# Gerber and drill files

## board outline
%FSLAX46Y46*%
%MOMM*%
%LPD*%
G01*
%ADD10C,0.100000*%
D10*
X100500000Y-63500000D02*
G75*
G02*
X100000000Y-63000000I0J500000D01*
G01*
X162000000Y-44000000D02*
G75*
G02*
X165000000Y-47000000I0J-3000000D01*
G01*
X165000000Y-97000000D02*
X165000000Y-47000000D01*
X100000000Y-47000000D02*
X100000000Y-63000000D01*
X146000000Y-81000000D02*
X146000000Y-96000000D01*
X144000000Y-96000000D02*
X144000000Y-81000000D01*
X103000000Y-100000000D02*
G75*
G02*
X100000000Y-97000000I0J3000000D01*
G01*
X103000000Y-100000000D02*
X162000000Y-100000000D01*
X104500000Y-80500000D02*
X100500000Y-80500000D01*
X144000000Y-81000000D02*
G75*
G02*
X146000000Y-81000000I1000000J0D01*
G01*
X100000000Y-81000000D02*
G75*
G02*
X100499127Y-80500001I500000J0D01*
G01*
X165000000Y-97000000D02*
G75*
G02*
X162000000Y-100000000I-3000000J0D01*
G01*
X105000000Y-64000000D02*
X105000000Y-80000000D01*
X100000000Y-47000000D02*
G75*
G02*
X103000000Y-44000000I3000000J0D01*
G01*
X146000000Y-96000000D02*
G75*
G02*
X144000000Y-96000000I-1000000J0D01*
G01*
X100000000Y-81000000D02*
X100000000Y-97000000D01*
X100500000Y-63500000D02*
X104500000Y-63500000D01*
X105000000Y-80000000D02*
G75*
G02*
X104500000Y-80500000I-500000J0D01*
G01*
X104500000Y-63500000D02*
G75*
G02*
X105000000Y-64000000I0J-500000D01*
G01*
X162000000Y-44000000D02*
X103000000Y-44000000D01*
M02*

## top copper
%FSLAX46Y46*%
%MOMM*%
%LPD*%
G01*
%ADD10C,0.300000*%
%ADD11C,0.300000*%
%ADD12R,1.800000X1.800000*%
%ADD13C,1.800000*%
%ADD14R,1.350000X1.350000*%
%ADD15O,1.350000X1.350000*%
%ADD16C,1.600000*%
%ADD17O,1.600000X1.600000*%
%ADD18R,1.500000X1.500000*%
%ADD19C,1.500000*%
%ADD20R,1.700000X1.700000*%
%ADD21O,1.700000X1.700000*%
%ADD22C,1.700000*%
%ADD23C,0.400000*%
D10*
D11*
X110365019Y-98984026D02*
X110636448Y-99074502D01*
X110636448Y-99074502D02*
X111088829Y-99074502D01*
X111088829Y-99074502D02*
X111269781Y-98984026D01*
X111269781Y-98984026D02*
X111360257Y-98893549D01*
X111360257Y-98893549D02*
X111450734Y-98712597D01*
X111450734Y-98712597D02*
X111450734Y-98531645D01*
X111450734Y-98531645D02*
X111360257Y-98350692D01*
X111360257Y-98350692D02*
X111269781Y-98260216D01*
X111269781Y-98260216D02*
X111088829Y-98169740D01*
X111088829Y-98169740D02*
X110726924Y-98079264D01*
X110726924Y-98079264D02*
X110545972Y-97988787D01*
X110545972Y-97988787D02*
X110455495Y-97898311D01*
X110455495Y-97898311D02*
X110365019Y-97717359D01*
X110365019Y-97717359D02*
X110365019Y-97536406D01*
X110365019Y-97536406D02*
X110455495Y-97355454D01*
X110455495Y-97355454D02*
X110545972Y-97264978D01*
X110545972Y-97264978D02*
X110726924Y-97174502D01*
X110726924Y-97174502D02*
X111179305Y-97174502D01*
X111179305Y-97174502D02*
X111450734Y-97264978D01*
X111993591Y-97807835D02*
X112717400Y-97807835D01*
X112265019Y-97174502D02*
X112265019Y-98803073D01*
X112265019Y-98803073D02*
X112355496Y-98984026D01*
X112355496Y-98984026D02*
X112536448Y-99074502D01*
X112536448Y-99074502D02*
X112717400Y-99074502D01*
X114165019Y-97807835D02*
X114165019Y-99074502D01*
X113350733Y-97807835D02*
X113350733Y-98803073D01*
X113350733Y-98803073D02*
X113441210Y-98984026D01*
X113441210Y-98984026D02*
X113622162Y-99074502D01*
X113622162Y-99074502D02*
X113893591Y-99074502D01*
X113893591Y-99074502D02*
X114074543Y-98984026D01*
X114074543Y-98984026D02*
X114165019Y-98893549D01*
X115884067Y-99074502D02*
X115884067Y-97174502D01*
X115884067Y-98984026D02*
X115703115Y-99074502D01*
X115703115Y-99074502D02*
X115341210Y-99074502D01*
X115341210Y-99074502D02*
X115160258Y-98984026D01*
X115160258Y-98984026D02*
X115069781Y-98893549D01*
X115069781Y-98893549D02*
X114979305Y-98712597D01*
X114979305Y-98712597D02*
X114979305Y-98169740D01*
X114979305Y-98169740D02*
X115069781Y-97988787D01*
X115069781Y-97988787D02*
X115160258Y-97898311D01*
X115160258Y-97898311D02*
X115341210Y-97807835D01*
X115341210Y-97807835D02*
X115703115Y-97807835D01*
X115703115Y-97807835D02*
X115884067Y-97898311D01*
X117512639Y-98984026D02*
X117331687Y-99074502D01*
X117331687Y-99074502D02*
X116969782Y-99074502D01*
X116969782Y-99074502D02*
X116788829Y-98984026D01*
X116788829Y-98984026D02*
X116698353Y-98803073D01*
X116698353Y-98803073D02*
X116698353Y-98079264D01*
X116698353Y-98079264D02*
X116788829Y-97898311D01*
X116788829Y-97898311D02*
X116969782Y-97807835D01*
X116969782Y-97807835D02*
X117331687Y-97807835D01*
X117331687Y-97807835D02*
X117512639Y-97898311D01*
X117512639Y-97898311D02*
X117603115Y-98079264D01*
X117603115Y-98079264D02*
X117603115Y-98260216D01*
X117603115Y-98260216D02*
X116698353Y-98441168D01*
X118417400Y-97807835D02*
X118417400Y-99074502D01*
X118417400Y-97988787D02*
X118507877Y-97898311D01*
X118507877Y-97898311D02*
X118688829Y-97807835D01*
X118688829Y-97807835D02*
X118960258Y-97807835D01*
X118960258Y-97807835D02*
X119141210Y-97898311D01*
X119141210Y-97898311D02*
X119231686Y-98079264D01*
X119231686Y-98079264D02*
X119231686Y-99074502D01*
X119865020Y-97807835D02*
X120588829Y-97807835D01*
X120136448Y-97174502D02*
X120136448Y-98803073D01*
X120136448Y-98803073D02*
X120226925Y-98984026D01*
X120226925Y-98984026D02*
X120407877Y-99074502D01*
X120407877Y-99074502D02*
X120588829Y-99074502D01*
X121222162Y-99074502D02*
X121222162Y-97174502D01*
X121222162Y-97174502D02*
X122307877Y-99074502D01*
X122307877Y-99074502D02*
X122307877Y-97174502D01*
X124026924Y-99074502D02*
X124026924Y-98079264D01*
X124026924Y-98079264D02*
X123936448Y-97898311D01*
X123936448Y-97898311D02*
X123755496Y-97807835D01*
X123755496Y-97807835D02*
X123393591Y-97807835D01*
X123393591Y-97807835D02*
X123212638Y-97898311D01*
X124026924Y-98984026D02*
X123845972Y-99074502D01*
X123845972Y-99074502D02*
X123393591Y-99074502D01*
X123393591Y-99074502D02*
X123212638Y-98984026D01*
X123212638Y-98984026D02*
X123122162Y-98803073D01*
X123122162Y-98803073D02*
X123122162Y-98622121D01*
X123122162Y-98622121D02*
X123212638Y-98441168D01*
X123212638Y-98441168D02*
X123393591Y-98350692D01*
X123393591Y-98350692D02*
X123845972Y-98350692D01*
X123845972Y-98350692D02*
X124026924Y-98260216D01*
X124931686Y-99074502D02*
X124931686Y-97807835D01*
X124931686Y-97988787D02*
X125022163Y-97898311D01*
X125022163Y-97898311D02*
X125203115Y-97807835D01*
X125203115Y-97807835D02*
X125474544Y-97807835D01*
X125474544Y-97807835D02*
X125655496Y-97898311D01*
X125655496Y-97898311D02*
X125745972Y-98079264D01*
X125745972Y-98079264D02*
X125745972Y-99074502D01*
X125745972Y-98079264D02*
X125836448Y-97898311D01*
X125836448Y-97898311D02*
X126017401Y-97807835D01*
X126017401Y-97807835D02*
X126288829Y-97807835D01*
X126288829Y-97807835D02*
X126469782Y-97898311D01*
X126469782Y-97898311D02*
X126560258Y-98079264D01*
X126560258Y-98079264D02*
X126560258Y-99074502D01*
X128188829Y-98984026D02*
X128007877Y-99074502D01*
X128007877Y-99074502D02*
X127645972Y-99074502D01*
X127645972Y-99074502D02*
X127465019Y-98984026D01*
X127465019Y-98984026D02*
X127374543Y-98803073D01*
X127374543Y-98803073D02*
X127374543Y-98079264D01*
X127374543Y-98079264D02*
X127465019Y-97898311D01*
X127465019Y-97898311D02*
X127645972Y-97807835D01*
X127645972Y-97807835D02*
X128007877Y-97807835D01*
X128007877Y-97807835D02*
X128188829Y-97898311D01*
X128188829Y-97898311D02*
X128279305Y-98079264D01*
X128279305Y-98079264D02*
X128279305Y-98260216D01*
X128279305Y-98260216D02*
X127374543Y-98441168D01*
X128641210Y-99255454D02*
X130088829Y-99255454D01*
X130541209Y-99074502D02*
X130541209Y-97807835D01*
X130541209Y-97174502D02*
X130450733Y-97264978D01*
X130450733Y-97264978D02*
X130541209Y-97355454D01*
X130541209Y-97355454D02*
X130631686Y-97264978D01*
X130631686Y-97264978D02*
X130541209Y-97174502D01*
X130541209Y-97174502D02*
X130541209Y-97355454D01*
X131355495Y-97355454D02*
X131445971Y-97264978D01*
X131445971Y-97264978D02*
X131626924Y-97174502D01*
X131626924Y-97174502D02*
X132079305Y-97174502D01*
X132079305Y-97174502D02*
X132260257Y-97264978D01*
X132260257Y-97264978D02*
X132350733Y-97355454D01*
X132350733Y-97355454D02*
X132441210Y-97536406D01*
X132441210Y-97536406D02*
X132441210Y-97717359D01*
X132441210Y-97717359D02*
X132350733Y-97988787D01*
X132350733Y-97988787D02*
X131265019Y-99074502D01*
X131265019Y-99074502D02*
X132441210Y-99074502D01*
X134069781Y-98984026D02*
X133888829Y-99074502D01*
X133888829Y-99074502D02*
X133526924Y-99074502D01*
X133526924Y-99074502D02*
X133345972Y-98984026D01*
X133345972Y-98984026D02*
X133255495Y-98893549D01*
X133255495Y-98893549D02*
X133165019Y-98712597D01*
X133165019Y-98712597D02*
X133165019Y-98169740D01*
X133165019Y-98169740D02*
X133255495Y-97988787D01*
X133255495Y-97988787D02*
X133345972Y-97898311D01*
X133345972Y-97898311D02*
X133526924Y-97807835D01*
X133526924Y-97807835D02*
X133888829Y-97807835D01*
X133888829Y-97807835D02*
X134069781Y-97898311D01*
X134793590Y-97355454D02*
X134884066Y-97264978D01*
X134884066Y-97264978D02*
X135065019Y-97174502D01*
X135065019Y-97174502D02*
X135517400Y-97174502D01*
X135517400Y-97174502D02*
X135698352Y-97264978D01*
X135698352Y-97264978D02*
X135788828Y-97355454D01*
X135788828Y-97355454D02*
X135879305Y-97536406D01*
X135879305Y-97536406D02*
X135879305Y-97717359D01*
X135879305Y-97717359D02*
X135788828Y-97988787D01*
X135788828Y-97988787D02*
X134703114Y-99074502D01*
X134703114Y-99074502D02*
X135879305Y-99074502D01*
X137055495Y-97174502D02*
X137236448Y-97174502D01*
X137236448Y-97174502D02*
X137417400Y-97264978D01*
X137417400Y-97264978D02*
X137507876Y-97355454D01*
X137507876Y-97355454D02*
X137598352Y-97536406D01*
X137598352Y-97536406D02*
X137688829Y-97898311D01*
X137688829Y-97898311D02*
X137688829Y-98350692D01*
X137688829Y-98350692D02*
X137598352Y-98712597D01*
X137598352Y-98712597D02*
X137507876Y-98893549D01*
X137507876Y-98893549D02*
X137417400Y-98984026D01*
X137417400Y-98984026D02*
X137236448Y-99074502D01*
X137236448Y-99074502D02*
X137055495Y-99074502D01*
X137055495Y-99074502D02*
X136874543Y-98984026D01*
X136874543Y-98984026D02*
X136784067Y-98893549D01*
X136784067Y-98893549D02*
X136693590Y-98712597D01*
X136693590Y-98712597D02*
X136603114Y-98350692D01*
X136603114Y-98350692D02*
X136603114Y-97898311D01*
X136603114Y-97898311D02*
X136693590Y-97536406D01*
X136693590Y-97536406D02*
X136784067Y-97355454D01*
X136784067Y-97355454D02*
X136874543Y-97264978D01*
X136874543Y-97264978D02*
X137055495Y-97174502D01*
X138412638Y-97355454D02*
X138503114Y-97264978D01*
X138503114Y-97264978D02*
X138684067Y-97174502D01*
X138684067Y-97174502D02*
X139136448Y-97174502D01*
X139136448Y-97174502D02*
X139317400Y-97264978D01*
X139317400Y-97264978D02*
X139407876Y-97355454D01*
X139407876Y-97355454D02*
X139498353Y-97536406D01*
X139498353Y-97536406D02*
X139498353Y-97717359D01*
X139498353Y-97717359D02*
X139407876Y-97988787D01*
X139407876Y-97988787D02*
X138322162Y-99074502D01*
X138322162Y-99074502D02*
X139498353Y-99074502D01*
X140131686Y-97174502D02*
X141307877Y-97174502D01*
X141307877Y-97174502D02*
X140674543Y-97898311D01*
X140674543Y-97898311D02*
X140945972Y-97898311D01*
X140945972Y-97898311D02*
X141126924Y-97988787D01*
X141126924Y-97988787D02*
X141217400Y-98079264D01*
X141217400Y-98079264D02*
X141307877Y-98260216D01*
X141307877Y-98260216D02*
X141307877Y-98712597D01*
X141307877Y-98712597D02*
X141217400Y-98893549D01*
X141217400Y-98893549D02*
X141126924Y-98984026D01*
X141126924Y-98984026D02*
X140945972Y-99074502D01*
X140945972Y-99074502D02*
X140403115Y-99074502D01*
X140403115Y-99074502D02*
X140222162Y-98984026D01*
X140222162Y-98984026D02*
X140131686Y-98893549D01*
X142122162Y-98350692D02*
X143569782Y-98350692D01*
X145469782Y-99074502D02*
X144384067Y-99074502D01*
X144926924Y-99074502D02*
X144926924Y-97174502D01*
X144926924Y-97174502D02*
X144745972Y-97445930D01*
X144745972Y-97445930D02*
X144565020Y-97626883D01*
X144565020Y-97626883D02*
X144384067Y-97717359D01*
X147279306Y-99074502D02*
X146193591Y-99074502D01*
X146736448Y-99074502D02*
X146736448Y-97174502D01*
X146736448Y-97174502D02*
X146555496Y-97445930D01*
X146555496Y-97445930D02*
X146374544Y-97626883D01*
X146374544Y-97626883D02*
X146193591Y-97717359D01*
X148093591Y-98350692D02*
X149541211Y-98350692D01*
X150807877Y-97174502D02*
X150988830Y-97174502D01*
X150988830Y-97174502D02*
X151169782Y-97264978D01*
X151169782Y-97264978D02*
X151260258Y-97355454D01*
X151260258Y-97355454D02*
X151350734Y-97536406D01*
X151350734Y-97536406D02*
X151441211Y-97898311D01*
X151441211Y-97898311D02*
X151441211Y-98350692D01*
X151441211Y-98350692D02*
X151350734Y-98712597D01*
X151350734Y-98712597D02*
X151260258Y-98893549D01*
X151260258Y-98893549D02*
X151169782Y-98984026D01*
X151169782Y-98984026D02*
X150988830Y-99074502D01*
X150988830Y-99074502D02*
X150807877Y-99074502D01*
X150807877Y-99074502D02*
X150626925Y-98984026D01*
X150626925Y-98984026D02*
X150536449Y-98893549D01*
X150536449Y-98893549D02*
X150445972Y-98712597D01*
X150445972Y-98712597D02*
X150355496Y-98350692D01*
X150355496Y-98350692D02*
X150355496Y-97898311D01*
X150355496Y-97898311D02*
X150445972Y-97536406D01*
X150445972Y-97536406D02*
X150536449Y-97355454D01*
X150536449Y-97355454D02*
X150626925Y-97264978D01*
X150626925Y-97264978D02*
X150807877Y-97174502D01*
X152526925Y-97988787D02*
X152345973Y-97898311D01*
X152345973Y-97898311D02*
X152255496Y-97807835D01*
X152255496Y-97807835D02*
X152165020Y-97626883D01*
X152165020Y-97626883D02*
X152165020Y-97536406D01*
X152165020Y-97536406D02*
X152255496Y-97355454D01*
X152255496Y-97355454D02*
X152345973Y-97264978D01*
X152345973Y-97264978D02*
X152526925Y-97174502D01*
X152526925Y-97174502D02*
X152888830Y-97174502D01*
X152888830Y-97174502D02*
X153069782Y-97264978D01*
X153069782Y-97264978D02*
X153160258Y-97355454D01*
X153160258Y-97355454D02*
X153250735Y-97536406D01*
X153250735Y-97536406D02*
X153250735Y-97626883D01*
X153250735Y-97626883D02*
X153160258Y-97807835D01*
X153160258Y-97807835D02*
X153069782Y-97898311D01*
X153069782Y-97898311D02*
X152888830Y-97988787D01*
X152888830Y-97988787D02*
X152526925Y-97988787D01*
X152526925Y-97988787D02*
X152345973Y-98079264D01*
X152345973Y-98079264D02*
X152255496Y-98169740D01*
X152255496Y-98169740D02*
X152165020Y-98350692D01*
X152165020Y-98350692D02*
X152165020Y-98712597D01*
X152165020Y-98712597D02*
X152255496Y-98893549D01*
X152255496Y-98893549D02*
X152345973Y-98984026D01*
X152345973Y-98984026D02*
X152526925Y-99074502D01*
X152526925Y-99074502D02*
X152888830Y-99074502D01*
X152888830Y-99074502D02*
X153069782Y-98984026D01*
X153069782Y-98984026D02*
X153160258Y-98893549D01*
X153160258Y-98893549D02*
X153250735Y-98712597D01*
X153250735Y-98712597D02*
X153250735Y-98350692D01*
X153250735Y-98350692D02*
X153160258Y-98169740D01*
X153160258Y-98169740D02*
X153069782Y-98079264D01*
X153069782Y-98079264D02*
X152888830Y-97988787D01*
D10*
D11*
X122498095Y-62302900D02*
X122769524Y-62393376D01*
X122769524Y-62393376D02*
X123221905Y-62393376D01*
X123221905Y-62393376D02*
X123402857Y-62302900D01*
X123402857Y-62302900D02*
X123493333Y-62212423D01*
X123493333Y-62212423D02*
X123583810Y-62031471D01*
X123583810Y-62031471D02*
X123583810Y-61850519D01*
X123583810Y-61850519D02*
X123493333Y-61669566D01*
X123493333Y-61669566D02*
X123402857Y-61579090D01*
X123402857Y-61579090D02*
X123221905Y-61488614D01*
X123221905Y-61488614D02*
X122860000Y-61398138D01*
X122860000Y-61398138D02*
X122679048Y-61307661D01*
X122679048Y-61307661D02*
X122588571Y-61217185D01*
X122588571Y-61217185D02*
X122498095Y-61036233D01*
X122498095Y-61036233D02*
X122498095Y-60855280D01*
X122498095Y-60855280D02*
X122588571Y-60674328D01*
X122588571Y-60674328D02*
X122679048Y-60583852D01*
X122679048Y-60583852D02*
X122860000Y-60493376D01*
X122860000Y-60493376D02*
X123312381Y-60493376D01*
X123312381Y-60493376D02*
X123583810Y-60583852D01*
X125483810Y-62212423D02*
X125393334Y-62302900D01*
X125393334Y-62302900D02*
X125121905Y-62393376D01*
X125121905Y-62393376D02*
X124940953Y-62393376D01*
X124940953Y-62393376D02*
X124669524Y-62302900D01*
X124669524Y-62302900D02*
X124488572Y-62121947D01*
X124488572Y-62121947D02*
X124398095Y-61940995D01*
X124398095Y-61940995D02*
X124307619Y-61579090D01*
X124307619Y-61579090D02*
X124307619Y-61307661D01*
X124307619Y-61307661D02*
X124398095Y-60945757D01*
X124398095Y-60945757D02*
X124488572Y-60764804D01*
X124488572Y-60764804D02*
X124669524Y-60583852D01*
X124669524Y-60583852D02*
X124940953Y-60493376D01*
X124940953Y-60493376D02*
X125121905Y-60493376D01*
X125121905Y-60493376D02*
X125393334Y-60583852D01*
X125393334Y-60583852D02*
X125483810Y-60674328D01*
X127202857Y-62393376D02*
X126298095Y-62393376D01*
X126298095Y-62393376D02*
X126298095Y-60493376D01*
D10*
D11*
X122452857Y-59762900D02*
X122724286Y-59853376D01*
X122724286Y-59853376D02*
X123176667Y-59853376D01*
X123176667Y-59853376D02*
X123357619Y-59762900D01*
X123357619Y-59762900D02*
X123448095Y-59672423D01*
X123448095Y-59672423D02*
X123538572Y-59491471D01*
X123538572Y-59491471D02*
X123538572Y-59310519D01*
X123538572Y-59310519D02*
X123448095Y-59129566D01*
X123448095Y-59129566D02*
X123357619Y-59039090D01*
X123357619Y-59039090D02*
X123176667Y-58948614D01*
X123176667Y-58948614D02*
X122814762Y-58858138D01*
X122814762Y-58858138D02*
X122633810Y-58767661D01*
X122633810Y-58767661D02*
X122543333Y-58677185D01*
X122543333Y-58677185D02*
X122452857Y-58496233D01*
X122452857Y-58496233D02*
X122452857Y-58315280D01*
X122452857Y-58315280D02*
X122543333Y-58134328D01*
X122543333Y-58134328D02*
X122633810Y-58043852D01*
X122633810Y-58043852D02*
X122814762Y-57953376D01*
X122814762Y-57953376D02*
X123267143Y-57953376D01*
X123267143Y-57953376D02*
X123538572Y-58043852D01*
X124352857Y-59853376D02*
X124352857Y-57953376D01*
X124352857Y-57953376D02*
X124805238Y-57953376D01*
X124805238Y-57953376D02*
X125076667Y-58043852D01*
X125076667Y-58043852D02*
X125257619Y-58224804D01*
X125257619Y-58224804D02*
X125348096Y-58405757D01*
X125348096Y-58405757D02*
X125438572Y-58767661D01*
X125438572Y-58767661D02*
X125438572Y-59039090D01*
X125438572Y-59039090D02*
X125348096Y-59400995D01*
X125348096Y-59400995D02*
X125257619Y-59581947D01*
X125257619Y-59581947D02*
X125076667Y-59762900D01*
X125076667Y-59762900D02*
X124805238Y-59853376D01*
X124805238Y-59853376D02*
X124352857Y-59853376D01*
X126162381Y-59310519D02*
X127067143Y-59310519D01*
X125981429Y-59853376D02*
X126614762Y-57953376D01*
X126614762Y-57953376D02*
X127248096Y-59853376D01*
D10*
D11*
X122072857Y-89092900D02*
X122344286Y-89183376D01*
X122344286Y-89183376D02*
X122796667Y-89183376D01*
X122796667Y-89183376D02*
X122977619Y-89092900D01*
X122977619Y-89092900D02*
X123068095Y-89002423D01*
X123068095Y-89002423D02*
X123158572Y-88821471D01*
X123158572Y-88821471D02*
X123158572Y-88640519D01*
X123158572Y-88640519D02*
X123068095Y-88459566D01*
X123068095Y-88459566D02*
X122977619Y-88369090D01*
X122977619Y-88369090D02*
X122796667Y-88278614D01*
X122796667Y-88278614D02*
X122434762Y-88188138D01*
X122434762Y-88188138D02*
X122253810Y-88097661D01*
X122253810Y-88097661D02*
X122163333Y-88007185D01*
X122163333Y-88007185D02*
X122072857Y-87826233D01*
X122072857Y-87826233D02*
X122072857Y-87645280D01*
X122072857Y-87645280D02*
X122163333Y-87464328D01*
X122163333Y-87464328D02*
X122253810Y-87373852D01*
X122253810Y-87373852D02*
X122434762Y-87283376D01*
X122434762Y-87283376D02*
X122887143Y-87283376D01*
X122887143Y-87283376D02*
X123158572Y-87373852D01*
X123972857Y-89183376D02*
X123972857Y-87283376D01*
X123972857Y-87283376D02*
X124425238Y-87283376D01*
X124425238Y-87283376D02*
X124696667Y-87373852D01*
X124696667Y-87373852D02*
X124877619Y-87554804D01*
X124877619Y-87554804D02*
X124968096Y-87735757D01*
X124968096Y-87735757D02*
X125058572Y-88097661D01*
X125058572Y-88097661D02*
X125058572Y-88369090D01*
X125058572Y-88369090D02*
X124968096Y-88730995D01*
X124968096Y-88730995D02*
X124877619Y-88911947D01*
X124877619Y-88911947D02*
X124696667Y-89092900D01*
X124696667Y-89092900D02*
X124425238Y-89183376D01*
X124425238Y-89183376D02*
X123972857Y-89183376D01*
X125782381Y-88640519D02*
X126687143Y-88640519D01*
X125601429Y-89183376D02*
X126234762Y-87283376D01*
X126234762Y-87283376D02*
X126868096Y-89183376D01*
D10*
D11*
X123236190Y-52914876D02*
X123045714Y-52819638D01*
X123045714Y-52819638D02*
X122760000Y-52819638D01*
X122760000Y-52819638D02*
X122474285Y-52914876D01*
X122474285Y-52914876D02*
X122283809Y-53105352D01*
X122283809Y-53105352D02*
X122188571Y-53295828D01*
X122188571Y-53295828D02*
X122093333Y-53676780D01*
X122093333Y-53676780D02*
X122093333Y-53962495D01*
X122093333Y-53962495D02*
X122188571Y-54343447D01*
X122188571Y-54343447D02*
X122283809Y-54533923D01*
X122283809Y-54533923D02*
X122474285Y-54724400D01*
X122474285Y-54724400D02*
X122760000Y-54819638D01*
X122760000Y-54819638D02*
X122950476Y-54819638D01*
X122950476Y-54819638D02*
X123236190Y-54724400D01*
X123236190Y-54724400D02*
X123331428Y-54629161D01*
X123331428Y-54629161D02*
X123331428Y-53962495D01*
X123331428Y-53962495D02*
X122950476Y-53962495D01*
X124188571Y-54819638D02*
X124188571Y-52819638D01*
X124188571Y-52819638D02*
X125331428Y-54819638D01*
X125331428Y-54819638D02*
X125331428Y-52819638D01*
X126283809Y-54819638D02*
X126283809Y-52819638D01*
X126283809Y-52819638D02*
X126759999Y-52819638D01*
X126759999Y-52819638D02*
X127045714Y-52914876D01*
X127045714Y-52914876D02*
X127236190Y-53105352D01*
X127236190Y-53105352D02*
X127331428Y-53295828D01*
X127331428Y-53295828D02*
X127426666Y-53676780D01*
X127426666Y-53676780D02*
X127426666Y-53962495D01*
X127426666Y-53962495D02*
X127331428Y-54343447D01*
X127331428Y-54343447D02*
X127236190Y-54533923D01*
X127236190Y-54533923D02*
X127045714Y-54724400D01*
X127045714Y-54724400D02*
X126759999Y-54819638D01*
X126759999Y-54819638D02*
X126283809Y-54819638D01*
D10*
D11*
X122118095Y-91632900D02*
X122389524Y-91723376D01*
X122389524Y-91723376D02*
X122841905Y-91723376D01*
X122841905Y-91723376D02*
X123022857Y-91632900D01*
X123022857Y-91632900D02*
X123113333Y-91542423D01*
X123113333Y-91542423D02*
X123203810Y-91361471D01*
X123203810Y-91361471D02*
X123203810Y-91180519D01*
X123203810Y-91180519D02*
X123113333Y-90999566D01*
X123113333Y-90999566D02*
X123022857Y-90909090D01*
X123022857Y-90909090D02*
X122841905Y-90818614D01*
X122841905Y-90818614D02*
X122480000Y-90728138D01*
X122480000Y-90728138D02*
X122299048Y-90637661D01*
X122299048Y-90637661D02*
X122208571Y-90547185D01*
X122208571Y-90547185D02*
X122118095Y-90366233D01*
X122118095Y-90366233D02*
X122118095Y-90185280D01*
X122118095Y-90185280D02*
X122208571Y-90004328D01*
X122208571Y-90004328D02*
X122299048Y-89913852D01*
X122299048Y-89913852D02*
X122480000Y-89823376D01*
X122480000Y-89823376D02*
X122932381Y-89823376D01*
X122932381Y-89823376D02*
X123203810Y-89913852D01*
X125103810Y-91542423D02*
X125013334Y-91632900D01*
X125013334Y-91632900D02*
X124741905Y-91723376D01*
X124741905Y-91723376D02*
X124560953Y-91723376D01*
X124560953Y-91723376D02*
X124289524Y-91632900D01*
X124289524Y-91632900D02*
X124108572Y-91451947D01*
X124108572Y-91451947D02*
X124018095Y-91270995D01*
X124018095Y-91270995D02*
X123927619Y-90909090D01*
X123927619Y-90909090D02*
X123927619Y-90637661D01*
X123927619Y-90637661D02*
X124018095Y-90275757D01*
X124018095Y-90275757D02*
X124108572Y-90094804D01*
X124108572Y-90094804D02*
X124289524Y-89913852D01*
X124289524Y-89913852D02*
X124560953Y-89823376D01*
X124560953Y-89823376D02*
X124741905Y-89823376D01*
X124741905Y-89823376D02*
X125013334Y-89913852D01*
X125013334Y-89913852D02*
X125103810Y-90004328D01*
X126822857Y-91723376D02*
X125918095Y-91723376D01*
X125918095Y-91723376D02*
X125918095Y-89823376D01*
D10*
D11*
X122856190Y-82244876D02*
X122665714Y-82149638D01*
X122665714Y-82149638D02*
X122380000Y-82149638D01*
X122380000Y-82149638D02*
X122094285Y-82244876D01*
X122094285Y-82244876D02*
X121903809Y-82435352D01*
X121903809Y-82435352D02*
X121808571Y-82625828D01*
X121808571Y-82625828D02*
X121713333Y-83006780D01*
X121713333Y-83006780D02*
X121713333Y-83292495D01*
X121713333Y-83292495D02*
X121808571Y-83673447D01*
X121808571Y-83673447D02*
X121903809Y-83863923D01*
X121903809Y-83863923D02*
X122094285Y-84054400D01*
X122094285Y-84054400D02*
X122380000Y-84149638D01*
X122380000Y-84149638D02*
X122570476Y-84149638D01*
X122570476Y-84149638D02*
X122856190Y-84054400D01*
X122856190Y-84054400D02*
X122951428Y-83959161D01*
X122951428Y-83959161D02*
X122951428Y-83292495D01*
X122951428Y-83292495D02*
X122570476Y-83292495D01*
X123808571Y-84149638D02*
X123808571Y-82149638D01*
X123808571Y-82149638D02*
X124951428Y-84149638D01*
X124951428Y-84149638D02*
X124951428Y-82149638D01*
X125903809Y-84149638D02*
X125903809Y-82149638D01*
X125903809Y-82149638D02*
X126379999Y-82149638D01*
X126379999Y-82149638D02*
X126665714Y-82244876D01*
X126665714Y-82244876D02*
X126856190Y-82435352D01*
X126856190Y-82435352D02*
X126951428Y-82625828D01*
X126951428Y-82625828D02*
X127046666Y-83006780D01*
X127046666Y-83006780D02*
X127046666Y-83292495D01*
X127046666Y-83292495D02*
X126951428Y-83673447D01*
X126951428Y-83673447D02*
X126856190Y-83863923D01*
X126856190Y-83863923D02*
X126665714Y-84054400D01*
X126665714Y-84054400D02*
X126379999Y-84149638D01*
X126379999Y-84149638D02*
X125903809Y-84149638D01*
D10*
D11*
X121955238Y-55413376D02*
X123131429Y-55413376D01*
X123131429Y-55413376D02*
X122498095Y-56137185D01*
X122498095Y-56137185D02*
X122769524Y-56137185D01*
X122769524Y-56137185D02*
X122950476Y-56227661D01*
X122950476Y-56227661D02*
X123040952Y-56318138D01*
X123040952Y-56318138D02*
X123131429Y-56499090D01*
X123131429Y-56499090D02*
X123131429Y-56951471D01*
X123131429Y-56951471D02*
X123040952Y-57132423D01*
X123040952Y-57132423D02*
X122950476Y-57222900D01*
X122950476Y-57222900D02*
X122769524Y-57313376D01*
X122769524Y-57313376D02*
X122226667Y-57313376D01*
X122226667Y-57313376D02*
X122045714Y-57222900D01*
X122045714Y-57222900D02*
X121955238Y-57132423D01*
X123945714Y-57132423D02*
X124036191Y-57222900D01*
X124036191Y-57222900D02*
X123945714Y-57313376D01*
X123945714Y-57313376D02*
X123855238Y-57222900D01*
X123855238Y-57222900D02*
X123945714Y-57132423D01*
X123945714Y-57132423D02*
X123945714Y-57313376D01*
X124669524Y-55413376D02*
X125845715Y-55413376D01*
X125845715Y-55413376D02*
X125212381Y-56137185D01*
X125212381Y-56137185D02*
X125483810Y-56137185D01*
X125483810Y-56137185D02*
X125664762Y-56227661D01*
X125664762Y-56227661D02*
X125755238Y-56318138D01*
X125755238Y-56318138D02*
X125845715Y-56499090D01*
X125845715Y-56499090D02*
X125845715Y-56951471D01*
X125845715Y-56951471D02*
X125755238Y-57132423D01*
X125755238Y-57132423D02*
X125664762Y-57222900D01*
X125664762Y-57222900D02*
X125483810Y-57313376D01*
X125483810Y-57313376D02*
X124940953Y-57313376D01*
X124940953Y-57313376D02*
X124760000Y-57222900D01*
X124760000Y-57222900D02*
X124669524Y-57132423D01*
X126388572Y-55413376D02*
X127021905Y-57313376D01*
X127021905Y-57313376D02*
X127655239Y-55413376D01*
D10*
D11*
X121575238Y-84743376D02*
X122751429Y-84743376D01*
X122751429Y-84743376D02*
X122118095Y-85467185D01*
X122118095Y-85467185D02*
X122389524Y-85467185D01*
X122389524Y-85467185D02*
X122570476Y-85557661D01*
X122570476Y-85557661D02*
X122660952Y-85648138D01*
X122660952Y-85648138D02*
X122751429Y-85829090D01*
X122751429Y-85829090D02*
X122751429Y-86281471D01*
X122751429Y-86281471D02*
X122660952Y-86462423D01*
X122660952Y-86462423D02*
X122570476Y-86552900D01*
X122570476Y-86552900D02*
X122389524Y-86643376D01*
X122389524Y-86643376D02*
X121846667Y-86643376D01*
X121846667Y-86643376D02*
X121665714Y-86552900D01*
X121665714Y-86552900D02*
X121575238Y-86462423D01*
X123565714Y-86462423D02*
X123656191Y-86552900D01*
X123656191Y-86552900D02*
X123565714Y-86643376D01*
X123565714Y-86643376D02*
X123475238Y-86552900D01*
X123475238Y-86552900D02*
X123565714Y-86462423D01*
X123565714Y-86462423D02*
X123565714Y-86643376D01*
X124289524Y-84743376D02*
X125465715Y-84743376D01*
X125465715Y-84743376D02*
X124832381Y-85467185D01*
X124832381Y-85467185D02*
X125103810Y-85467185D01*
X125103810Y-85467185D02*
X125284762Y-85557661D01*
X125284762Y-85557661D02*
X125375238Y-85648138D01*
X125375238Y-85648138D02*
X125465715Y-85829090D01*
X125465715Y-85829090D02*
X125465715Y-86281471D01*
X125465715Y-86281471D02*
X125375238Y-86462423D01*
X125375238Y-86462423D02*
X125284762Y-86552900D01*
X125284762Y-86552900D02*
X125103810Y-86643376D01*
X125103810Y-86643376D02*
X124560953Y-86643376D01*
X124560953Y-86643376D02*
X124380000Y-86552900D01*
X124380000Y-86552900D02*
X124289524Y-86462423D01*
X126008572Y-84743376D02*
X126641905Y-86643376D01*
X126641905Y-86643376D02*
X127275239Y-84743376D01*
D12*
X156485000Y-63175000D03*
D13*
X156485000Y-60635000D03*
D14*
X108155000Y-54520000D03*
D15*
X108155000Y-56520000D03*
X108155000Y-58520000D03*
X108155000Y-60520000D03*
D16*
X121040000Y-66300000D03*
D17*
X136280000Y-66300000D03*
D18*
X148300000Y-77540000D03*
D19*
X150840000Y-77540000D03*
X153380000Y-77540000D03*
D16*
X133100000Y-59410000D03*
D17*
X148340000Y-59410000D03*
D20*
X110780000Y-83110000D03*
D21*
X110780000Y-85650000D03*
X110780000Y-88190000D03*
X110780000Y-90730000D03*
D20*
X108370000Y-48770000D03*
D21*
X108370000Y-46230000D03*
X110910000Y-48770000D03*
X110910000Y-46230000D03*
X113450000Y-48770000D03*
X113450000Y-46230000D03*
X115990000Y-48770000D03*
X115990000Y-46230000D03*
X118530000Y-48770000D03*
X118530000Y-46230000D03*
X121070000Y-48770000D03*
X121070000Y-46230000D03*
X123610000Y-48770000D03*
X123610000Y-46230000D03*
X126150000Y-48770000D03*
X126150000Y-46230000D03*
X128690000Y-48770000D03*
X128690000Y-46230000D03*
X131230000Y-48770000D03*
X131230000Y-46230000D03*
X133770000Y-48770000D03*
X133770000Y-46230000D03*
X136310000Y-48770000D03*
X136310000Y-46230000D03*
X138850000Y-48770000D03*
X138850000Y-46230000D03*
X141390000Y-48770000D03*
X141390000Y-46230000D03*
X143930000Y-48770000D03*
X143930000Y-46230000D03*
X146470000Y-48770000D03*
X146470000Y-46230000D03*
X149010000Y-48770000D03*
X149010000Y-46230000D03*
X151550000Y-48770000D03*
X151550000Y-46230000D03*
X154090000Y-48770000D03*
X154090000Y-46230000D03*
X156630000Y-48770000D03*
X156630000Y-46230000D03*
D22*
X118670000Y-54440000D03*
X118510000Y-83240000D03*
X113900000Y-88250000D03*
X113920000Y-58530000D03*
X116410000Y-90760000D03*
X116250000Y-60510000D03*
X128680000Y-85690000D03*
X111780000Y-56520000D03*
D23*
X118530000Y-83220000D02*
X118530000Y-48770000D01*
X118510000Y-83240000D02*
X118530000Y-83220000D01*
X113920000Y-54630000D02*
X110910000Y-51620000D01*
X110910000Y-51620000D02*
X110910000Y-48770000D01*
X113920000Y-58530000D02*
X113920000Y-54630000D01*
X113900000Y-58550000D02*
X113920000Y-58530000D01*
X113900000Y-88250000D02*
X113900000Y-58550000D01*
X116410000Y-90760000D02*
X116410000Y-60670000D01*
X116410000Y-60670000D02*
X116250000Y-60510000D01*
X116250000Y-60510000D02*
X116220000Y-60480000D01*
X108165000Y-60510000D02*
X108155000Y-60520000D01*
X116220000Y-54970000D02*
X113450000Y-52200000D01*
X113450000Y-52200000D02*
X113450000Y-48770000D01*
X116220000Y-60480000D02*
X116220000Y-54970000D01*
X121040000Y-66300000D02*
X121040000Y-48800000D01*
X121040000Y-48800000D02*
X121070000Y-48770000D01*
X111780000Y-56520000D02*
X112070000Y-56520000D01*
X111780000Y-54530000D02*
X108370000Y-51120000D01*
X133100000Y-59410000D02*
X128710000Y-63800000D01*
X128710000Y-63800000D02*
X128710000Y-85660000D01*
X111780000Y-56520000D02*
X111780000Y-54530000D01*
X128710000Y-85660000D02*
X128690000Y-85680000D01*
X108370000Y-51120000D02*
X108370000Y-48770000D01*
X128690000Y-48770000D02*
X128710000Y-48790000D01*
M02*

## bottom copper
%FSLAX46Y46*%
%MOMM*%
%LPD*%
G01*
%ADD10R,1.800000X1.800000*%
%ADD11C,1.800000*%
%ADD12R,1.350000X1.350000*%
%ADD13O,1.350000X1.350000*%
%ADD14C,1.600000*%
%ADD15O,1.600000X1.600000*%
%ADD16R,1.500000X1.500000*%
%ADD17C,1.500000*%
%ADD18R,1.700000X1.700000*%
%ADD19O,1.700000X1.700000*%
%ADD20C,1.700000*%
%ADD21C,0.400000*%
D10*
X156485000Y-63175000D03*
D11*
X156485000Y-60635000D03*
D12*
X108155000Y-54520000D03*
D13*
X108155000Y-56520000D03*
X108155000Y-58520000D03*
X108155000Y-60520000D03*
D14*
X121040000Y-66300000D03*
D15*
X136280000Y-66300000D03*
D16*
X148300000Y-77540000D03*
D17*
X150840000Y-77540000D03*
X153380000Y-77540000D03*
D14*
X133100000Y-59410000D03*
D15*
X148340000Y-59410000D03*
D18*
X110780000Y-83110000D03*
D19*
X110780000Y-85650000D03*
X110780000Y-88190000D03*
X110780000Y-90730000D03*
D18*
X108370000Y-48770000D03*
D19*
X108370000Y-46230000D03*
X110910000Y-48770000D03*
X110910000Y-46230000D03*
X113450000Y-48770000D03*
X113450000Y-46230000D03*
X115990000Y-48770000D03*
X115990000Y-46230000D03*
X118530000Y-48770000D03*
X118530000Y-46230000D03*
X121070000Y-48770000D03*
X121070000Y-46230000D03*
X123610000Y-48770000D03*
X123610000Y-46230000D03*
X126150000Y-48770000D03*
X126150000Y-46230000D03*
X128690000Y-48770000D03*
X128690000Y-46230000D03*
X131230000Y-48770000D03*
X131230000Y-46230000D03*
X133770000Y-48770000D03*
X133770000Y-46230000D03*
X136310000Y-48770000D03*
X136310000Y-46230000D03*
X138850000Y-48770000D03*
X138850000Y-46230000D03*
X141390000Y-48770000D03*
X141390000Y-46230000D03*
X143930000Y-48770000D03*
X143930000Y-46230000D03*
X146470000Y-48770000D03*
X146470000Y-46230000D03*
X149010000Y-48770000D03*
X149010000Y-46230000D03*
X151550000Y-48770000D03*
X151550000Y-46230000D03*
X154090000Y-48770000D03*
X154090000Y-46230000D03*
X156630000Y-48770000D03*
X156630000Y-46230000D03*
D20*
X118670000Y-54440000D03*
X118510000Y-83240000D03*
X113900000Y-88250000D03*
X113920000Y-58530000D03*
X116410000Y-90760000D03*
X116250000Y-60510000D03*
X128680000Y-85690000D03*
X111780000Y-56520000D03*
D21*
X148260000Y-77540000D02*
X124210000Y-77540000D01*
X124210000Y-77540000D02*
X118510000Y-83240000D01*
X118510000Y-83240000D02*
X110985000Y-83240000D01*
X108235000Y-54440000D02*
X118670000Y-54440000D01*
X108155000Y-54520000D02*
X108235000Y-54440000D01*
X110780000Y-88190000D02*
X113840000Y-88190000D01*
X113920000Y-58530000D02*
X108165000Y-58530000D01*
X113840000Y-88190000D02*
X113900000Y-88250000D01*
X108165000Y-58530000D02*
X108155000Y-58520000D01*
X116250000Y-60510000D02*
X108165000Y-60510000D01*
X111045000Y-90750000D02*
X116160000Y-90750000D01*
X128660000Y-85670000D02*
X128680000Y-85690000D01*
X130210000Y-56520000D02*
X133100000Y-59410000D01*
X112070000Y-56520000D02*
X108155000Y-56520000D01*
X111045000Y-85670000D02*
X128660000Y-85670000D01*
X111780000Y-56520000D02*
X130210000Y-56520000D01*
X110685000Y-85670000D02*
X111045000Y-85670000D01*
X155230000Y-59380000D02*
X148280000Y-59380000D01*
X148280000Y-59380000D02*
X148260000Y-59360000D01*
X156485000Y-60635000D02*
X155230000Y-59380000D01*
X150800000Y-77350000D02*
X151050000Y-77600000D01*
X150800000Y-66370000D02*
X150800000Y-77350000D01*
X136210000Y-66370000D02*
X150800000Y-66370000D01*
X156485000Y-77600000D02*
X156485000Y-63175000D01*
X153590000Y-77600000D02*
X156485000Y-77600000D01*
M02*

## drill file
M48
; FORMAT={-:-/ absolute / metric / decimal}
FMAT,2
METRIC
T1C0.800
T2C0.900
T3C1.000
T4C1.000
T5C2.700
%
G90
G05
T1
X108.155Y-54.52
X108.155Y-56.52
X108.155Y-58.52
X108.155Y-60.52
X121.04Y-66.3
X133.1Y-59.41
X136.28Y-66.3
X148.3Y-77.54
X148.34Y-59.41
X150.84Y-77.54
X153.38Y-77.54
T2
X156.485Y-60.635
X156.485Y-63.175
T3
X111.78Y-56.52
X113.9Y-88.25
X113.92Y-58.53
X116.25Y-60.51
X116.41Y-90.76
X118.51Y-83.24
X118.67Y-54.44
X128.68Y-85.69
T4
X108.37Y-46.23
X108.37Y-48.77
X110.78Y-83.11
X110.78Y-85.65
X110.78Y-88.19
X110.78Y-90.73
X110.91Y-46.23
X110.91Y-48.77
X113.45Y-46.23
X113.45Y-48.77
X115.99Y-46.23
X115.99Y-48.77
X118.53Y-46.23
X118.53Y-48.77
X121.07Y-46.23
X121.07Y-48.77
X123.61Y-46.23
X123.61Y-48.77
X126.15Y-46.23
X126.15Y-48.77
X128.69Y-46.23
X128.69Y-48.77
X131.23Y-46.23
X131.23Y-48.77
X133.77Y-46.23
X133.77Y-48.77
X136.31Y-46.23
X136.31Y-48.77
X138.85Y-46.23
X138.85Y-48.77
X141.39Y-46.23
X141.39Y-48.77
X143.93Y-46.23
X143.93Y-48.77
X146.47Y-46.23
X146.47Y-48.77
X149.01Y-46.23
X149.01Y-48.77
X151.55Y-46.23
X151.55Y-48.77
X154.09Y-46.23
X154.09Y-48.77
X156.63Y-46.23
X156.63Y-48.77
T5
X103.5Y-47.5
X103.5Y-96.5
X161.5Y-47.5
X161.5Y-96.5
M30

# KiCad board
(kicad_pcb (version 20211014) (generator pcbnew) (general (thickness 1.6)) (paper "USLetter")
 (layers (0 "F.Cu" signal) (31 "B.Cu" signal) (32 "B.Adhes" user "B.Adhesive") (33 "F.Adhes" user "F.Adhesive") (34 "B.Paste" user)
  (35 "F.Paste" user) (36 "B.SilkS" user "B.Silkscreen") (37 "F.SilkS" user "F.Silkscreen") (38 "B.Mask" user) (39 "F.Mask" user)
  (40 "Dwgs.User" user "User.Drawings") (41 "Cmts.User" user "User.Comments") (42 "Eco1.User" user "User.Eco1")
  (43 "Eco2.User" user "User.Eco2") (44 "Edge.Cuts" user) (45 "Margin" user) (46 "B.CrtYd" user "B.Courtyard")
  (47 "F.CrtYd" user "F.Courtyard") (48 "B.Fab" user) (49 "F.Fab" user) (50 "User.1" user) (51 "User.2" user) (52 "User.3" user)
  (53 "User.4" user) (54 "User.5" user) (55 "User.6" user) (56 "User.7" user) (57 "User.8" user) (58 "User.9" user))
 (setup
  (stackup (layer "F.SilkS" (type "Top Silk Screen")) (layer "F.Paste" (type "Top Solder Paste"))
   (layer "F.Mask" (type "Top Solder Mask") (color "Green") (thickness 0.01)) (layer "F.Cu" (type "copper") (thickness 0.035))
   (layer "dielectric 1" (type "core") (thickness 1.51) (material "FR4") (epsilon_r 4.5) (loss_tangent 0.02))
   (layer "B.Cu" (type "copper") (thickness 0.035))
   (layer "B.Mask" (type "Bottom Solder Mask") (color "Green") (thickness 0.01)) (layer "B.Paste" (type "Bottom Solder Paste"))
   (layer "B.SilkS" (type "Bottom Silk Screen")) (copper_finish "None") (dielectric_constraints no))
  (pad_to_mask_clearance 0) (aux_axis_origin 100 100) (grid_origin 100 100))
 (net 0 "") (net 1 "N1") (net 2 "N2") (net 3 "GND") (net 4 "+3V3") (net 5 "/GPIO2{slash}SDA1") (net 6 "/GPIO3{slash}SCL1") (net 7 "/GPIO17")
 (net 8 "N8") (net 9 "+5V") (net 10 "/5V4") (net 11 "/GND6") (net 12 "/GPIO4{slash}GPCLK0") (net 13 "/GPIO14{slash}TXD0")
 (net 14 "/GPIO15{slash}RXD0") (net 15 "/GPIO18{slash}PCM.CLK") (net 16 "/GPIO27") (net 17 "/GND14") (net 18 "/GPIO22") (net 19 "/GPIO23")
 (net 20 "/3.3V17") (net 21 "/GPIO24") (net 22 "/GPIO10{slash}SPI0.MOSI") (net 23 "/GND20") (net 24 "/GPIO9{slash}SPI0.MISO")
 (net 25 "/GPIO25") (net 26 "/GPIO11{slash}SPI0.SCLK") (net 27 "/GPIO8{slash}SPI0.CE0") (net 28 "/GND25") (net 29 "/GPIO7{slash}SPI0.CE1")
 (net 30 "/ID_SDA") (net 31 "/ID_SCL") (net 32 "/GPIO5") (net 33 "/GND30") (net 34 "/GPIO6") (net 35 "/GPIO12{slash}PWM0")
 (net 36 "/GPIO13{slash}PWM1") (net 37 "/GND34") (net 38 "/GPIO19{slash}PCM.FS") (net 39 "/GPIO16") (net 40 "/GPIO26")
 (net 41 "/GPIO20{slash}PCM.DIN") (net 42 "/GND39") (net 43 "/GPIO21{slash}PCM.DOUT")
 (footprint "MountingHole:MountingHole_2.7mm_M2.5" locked (layer "F.Cu") (at 161.5 47.5)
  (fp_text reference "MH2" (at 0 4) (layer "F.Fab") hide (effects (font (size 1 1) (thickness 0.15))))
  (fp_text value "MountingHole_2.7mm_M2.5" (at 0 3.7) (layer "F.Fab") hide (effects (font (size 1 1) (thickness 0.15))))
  (pad "" np_thru_hole circle locked (at 0 0) (size 2.7 2.7) (drill 2.7) (layers *.Cu *.Mask)))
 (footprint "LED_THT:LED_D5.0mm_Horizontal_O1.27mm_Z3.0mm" (layer "F.Cu") (at 156.485 63.175 90)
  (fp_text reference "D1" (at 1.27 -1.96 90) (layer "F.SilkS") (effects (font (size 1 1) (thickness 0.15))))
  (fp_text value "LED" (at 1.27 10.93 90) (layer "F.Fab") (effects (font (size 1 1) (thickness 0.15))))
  (pad "1" thru_hole rect (at 0 0 90) (size 1.8 1.8) (drill 0.9) (layers *.Cu *.Mask) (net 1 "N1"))
  (pad "2" thru_hole circle (at 2.54 0 90) (size 1.8 1.8) (drill 0.9) (layers *.Cu *.Mask) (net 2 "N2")))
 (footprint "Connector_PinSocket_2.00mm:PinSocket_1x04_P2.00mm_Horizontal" (layer "F.Cu") (at 108.155 54.52)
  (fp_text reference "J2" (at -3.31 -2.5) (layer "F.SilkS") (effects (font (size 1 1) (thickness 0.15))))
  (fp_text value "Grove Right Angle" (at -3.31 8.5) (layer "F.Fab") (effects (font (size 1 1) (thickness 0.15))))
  (pad "1" thru_hole rect (at 0 0) (size 1.35 1.35) (drill 0.8) (layers *.Cu *.Mask) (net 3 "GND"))
  (pad "2" thru_hole oval (at 0 2) (size 1.35 1.35) (drill 0.8) (layers *.Cu *.Mask) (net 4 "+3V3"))
  (pad "3" thru_hole oval (at 0 4) (size 1.35 1.35) (drill 0.8) (layers *.Cu *.Mask) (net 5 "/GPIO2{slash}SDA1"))
  (pad "4" thru_hole oval (at 0 6) (size 1.35 1.35) (drill 0.8) (layers *.Cu *.Mask) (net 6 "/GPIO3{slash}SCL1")))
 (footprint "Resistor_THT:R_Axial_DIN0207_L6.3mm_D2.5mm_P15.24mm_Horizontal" (layer "F.Cu") (at 121.04 66.3)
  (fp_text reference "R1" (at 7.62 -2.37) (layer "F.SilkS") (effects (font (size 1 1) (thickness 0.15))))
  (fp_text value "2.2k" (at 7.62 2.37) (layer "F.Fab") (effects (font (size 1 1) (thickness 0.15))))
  (pad "1" thru_hole circle (at 0 0) (size 1.6 1.6) (drill 0.8) (layers *.Cu *.Mask) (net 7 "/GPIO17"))
  (pad "2" thru_hole oval (at 15.24 0) (size 1.6 1.6) (drill 0.8) (layers *.Cu *.Mask) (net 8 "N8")))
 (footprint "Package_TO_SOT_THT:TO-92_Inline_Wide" (layer "F.Cu") (at 148.3 77.54)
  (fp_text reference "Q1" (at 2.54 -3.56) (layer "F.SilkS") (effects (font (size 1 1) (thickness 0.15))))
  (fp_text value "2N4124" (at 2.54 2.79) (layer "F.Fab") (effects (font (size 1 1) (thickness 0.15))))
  (pad "1" thru_hole rect (at 0 0) (size 1.5 1.5) (drill 0.8) (layers *.Cu *.Mask) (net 3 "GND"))
  (pad "2" thru_hole circle (at 2.54 0) (size 1.5 1.5) (drill 0.8) (layers *.Cu *.Mask) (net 8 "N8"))
  (pad "3" thru_hole circle (at 5.08 0) (size 1.5 1.5) (drill 0.8) (layers *.Cu *.Mask) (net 1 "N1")))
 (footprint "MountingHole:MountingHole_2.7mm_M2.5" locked (layer "F.Cu") (at 103.5 96.5)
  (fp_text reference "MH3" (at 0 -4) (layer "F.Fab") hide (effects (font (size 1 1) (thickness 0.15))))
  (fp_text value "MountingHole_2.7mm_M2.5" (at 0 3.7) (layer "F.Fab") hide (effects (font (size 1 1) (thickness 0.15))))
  (pad "" np_thru_hole circle locked (at 0 0) (size 2.7 2.7) (drill 2.7) (layers *.Cu *.Mask)))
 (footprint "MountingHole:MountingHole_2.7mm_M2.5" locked (layer "F.Cu") (at 103.5 47.5)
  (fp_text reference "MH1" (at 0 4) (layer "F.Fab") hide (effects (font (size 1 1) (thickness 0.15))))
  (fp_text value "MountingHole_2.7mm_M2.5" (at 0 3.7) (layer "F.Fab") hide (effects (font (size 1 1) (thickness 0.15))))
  (pad "" np_thru_hole circle locked (at 0 0) (size 2.7 2.7) (drill 2.7) (layers *.Cu *.Mask)))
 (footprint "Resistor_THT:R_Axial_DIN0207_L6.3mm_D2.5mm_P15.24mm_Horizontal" (layer "F.Cu") (at 133.1 59.41)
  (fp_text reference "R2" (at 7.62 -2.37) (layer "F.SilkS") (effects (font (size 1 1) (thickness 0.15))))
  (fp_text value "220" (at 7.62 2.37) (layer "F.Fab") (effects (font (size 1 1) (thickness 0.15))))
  (pad "1" thru_hole circle (at 0 0) (size 1.6 1.6) (drill 0.8) (layers *.Cu *.Mask) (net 4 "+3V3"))
  (pad "2" thru_hole oval (at 15.24 0) (size 1.6 1.6) (drill 0.8) (layers *.Cu *.Mask) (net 2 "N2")))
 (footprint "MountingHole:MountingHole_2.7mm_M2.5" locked (layer "F.Cu") (at 161.5 96.5)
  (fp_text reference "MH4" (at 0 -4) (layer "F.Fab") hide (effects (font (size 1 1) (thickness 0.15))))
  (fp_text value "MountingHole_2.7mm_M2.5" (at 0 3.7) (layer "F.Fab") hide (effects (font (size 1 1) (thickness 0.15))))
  (pad "" np_thru_hole circle locked (at 0 0) (size 2.7 2.7) (drill 2.7) (layers *.Cu *.Mask)))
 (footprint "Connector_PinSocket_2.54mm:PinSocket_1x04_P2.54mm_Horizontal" (layer "F.Cu") (at 110.78 83.11)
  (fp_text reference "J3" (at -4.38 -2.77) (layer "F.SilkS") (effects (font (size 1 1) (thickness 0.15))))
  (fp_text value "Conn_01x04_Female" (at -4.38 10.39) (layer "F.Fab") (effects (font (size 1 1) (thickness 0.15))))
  (pad "1" thru_hole rect (at 0 0) (size 1.7 1.7) (drill 1) (layers *.Cu *.Mask) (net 3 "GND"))
  (pad "2" thru_hole oval (at 0 2.54) (size 1.7 1.7) (drill 1) (layers *.Cu *.Mask) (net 4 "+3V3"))
  (pad "3" thru_hole oval (at 0 5.08) (size 1.7 1.7) (drill 1) (layers *.Cu *.Mask) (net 5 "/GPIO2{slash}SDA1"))
  (pad "4" thru_hole oval (at 0 7.62) (size 1.7 1.7) (drill 1) (layers *.Cu *.Mask) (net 6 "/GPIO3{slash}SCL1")))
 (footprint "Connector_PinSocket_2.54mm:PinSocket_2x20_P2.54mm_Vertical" (layer "B.Cu") (at 108.37 48.77 -90)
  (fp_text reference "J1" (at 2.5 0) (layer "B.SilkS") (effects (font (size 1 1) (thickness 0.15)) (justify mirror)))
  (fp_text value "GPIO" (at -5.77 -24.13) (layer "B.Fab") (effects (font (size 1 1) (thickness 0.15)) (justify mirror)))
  (pad "1" thru_hole rect (at 0 0 270) (size 1.7 1.7) (drill 1) (layers *.Cu *.Mask) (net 4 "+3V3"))
  (pad "2" thru_hole oval (at -2.54 0 270) (size 1.7 1.7) (drill 1) (layers *.Cu *.Mask) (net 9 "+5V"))
  (pad "3" thru_hole oval (at 0 -2.54 270) (size 1.7 1.7) (drill 1) (layers *.Cu *.Mask) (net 5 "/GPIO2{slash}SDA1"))
  (pad "4" thru_hole oval (at -2.54 -2.54 270) (size 1.7 1.7) (drill 1) (layers *.Cu *.Mask) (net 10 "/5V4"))
  (pad "5" thru_hole oval (at 0 -5.08 270) (size 1.7 1.7) (drill 1) (layers *.Cu *.Mask) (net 6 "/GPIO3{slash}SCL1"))
  (pad "6" thru_hole oval (at -2.54 -5.08 270) (size 1.7 1.7) (drill 1) (layers *.Cu *.Mask) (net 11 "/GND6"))
  (pad "7" thru_hole oval (at 0 -7.62 270) (size 1.7 1.7) (drill 1) (layers *.Cu *.Mask) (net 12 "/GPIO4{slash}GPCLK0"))
  (pad "8" thru_hole oval (at -2.54 -7.62 270) (size 1.7 1.7) (drill 1) (layers *.Cu *.Mask) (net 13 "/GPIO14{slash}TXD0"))
  (pad "9" thru_hole oval (at 0 -10.16 270) (size 1.7 1.7) (drill 1) (layers *.Cu *.Mask) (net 3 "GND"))
  (pad "10" thru_hole oval (at -2.54 -10.16 270) (size 1.7 1.7) (drill 1) (layers *.Cu *.Mask) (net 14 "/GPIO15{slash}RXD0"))
  (pad "11" thru_hole oval (at 0 -12.7 270) (size 1.7 1.7) (drill 1) (layers *.Cu *.Mask) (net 7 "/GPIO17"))
  (pad "12" thru_hole oval (at -2.54 -12.7 270) (size 1.7 1.7) (drill 1) (layers *.Cu *.Mask) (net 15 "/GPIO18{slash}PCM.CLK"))
  (pad "13" thru_hole oval (at 0 -15.24 270) (size 1.7 1.7) (drill 1) (layers *.Cu *.Mask) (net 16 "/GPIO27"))
  (pad "14" thru_hole oval (at -2.54 -15.24 270) (size 1.7 1.7) (drill 1) (layers *.Cu *.Mask) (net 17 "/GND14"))
  (pad "15" thru_hole oval (at 0 -17.78 270) (size 1.7 1.7) (drill 1) (layers *.Cu *.Mask) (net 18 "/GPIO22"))
  (pad "16" thru_hole oval (at -2.54 -17.78 270) (size 1.7 1.7) (drill 1) (layers *.Cu *.Mask) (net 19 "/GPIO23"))
  (pad "17" thru_hole oval (at 0 -20.32 270) (size 1.7 1.7) (drill 1) (layers *.Cu *.Mask) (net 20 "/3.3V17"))
  (pad "18" thru_hole oval (at -2.54 -20.32 270) (size 1.7 1.7) (drill 1) (layers *.Cu *.Mask) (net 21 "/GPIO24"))
  (pad "19" thru_hole oval (at 0 -22.86 270) (size 1.7 1.7) (drill 1) (layers *.Cu *.Mask) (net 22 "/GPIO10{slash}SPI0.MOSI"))
  (pad "20" thru_hole oval (at -2.54 -22.86 270) (size 1.7 1.7) (drill 1) (layers *.Cu *.Mask) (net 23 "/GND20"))
  (pad "21" thru_hole oval (at 0 -25.4 270) (size 1.7 1.7) (drill 1) (layers *.Cu *.Mask) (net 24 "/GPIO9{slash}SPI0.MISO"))
  (pad "22" thru_hole oval (at -2.54 -25.4 270) (size 1.7 1.7) (drill 1) (layers *.Cu *.Mask) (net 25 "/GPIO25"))
  (pad "23" thru_hole oval (at 0 -27.94 270) (size 1.7 1.7) (drill 1) (layers *.Cu *.Mask) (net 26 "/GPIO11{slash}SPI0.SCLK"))
  (pad "24" thru_hole oval (at -2.54 -27.94 270) (size 1.7 1.7) (drill 1) (layers *.Cu *.Mask) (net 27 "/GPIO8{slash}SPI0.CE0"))
  (pad "25" thru_hole oval (at 0 -30.48 270) (size 1.7 1.7) (drill 1) (layers *.Cu *.Mask) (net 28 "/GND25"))
  (pad "26" thru_hole oval (at -2.54 -30.48 270) (size 1.7 1.7) (drill 1) (layers *.Cu *.Mask) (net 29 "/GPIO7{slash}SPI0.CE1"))
  (pad "27" thru_hole oval (at 0 -33.02 270) (size 1.7 1.7) (drill 1) (layers *.Cu *.Mask) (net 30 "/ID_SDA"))
  (pad "28" thru_hole oval (at -2.54 -33.02 270) (size 1.7 1.7) (drill 1) (layers *.Cu *.Mask) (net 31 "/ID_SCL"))
  (pad "29" thru_hole oval (at 0 -35.56 270) (size 1.7 1.7) (drill 1) (layers *.Cu *.Mask) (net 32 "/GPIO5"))
  (pad "30" thru_hole oval (at -2.54 -35.56 270) (size 1.7 1.7) (drill 1) (layers *.Cu *.Mask) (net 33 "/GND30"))
  (pad "31" thru_hole oval (at 0 -38.1 270) (size 1.7 1.7) (drill 1) (layers *.Cu *.Mask) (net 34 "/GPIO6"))
  (pad "32" thru_hole oval (at -2.54 -38.1 270) (size 1.7 1.7) (drill 1) (layers *.Cu *.Mask) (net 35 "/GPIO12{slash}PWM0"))
  (pad "33" thru_hole oval (at 0 -40.64 270) (size 1.7 1.7) (drill 1) (layers *.Cu *.Mask) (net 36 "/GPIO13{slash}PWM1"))
  (pad "34" thru_hole oval (at -2.54 -40.64 270) (size 1.7 1.7) (drill 1) (layers *.Cu *.Mask) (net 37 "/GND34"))
  (pad "35" thru_hole oval (at 0 -43.18 270) (size 1.7 1.7) (drill 1) (layers *.Cu *.Mask) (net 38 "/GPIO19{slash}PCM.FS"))
  (pad "36" thru_hole oval (at -2.54 -43.18 270) (size 1.7 1.7) (drill 1) (layers *.Cu *.Mask) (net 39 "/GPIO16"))
  (pad "37" thru_hole oval (at 0 -45.72 270) (size 1.7 1.7) (drill 1) (layers *.Cu *.Mask) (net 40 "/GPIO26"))
  (pad "38" thru_hole oval (at -2.54 -45.72 270) (size 1.7 1.7) (drill 1) (layers *.Cu *.Mask) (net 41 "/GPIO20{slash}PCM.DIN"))
  (pad "39" thru_hole oval (at 0 -48.26 270) (size 1.7 1.7) (drill 1) (layers *.Cu *.Mask) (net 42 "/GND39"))
  (pad "40" thru_hole oval (at -2.54 -48.26 270) (size 1.7 1.7) (drill 1) (layers *.Cu *.Mask) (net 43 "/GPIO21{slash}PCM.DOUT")))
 (gr_arc (start 100.5 63.5) (mid 100.146447 63.353553) (end 100 63) (layer "Edge.Cuts") (width 0.1))
 (gr_arc (start 162 44) (mid 164.12132 44.87868) (end 165 47) (layer "Edge.Cuts") (width 0.1))
 (gr_line (start 165 97) (end 165 47) (layer "Edge.Cuts") (width 0.1))
 (gr_line (start 100 47) (end 100 63) (layer "Edge.Cuts") (width 0.1))
 (gr_line (start 146 81) (end 146 96) (layer "Edge.Cuts") (width 0.1))
 (gr_line (start 144 96) (end 144 81) (layer "Edge.Cuts") (width 0.1))
 (gr_arc (start 103 100) (mid 100.87868 99.12132) (end 100 97) (layer "Edge.Cuts") (width 0.1))
 (gr_line (start 103 100) (end 162 100) (layer "Edge.Cuts") (width 0.1))
 (gr_line (start 104.5 80.5) (end 100.5 80.5) (layer "Edge.Cuts") (width 0.1))
 (gr_arc (start 144 81) (mid 145 80) (end 146 81) (layer "Edge.Cuts") (width 0.1))
 (gr_arc (start 100 81) (mid 100.146138 80.646755) (end 100.499127 80.500001) (layer "Edge.Cuts") (width 0.1))
 (gr_arc (start 165 97) (mid 164.12132 99.12132) (end 162 100) (layer "Edge.Cuts") (width 0.1))
 (gr_line (start 105 64) (end 105 80) (layer "Edge.Cuts") (width 0.1))
 (gr_arc (start 100 47) (mid 100.87868 44.87868) (end 103 44) (layer "Edge.Cuts") (width 0.1))
 (gr_arc (start 146 96) (mid 145 97) (end 144 96) (layer "Edge.Cuts") (width 0.1))
 (gr_line (start 100 81) (end 100 97) (layer "Edge.Cuts") (width 0.1))
 (gr_line (start 100.5 63.5) (end 104.5 63.5) (layer "Edge.Cuts") (width 0.1))
 (gr_arc (start 105 80) (mid 104.853553 80.353553) (end 104.5 80.5) (layer "Edge.Cuts") (width 0.1))
 (gr_arc (start 104.5 63.5) (mid 104.853553 63.646447) (end 105 64) (layer "Edge.Cuts") (width 0.1))
 (gr_line (start 162 44) (end 103 44) (layer "Edge.Cuts") (width 0.1))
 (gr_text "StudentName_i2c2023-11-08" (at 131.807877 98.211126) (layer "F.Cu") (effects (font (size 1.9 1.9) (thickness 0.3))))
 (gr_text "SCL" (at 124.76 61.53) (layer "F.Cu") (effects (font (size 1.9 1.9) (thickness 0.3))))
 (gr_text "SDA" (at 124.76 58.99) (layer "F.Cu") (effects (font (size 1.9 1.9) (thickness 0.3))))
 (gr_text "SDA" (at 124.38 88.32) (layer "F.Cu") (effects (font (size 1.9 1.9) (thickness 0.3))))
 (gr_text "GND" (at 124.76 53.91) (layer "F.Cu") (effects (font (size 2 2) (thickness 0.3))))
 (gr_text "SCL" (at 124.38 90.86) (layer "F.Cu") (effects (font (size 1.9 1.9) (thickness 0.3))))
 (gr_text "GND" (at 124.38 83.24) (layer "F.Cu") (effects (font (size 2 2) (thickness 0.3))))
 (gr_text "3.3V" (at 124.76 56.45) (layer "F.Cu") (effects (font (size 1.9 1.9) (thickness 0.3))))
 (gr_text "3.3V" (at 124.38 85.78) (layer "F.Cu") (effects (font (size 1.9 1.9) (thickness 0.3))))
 (segment (start 118.53 83.22) (end 118.53 48.77) (width 0.4) (layer "F.Cu") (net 3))
 (segment (start 118.51 83.24) (end 118.53 83.22) (width 0.4) (layer "F.Cu") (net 3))
 (via (at 118.67 54.44) (size 1.7) (drill 1) (layers "F.Cu" "B.Cu") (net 3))
 (via (at 118.51 83.24) (size 1.7) (drill 1) (layers "F.Cu" "B.Cu") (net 3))
 (segment (start 148.26 77.54) (end 124.21 77.54) (width 0.4) (layer "B.Cu") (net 3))
 (segment (start 124.21 77.54) (end 118.51 83.24) (width 0.4) (layer "B.Cu") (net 3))
 (segment (start 118.51 83.24) (end 110.985 83.24) (width 0.4) (layer "B.Cu") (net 3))
 (segment (start 108.235 54.44) (end 118.67 54.44) (width 0.4) (layer "B.Cu") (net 3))
 (segment (start 108.155 54.52) (end 108.235 54.44) (width 0.4) (layer "B.Cu") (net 3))
 (segment (start 113.92 54.63) (end 110.91 51.62) (width 0.4) (layer "F.Cu") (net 5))
 (segment (start 110.91 51.62) (end 110.91 48.77) (width 0.4) (layer "F.Cu") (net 5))
 (segment (start 113.92 58.53) (end 113.92 54.63) (width 0.4) (layer "F.Cu") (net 5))
 (segment (start 113.9 58.55) (end 113.92 58.53) (width 0.4) (layer "F.Cu") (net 5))
 (segment (start 113.9 88.25) (end 113.9 58.55) (width 0.4) (layer "F.Cu") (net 5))
 (via (at 113.9 88.25) (size 1.7) (drill 1) (layers "F.Cu" "B.Cu") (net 5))
 (via (at 113.92 58.53) (size 1.7) (drill 1) (layers "F.Cu" "B.Cu") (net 5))
 (segment (start 110.78 88.19) (end 113.84 88.19) (width 0.4) (layer "B.Cu") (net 5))
 (segment (start 113.92 58.53) (end 108.165 58.53) (width 0.4) (layer "B.Cu") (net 5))
 (segment (start 113.84 88.19) (end 113.9 88.25) (width 0.4) (layer "B.Cu") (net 5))
 (segment (start 108.165 58.53) (end 108.155 58.52) (width 0.4) (layer "B.Cu") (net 5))
 (segment (start 116.41 90.76) (end 116.41 60.67) (width 0.4) (layer "F.Cu") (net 6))
 (segment (start 116.41 60.67) (end 116.25 60.51) (width 0.4) (layer "F.Cu") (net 6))
 (segment (start 116.25 60.51) (end 116.22 60.48) (width 0.4) (layer "F.Cu") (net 6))
 (segment (start 108.165 60.51) (end 108.155 60.52) (width 0.4) (layer "F.Cu") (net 6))
 (segment (start 116.22 54.97) (end 113.45 52.2) (width 0.4) (layer "F.Cu") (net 6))
 (segment (start 113.45 52.2) (end 113.45 48.77) (width 0.4) (layer "F.Cu") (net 6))
 (segment (start 116.22 60.48) (end 116.22 54.97) (width 0.4) (layer "F.Cu") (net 6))
 (via (at 116.41 90.76) (size 1.7) (drill 1) (layers "F.Cu" "B.Cu") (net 6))
 (via (at 116.25 60.51) (size 1.7) (drill 1) (layers "F.Cu" "B.Cu") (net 6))
 (segment (start 116.25 60.51) (end 108.165 60.51) (width 0.4) (layer "B.Cu") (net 6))
 (segment (start 111.045 90.75) (end 116.16 90.75) (width 0.4) (layer "B.Cu") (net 6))
 (segment (start 121.04 66.3) (end 121.04 48.8) (width 0.4) (layer "F.Cu") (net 7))
 (segment (start 121.04 48.8) (end 121.07 48.77) (width 0.4) (layer "F.Cu") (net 7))
 (segment (start 111.78 56.52) (end 112.07 56.52) (width 0.4) (layer "F.Cu") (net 4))
 (segment (start 111.78 54.53) (end 108.37 51.12) (width 0.4) (layer "F.Cu") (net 4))
 (segment (start 133.1 59.41) (end 128.71 63.8) (width 0.4) (layer "F.Cu") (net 4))
 (segment (start 128.71 63.8) (end 128.71 85.66) (width 0.4) (layer "F.Cu") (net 4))
 (segment (start 111.78 56.52) (end 111.78 54.53) (width 0.4) (layer "F.Cu") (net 4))
 (segment (start 128.71 85.66) (end 128.69 85.68) (width 0.4) (layer "F.Cu") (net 4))
 (segment (start 108.37 51.12) (end 108.37 48.77) (width 0.4) (layer "F.Cu") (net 4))
 (via (at 128.68 85.69) (size 1.7) (drill 1) (layers "F.Cu" "B.Cu") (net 4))
 (via (at 111.78 56.52) (size 1.7) (drill 1) (layers "F.Cu" "B.Cu") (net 4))
 (segment (start 128.66 85.67) (end 128.68 85.69) (width 0.4) (layer "B.Cu") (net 4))
 (segment (start 130.21 56.52) (end 133.1 59.41) (width 0.4) (layer "B.Cu") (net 4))
 (segment (start 112.07 56.52) (end 108.155 56.52) (width 0.4) (layer "B.Cu") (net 4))
 (segment (start 111.045 85.67) (end 128.66 85.67) (width 0.4) (layer "B.Cu") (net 4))
 (segment (start 111.78 56.52) (end 130.21 56.52) (width 0.4) (layer "B.Cu") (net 4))
 (segment (start 110.685 85.67) (end 111.045 85.67) (width 0.4) (layer "B.Cu") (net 4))
 (segment (start 155.23 59.38) (end 148.28 59.38) (width 0.4) (layer "B.Cu") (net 2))
 (segment (start 148.28 59.38) (end 148.26 59.36) (width 0.4) (layer "B.Cu") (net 2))
 (segment (start 156.485 60.635) (end 155.23 59.38) (width 0.4) (layer "B.Cu") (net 2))
 (segment (start 150.8 77.35) (end 151.05 77.6) (width 0.4) (layer "B.Cu") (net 8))
 (segment (start 150.8 66.37) (end 150.8 77.35) (width 0.4) (layer "B.Cu") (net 8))
 (segment (start 136.21 66.37) (end 150.8 66.37) (width 0.4) (layer "B.Cu") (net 8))
 (segment (start 156.485 77.6) (end 156.485 63.175) (width 0.4) (layer "B.Cu") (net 1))
 (segment (start 153.59 77.6) (end 156.485 77.6) (width 0.4) (layer "B.Cu") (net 1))
 (segment (start 128.69 48.77) (end 128.71 48.79) (width 0.4) (layer "F.Cu") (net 20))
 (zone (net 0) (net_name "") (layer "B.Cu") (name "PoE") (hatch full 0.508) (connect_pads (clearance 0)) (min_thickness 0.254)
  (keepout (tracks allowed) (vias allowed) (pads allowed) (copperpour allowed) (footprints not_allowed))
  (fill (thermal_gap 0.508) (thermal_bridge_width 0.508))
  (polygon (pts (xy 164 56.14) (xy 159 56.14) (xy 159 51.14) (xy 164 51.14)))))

